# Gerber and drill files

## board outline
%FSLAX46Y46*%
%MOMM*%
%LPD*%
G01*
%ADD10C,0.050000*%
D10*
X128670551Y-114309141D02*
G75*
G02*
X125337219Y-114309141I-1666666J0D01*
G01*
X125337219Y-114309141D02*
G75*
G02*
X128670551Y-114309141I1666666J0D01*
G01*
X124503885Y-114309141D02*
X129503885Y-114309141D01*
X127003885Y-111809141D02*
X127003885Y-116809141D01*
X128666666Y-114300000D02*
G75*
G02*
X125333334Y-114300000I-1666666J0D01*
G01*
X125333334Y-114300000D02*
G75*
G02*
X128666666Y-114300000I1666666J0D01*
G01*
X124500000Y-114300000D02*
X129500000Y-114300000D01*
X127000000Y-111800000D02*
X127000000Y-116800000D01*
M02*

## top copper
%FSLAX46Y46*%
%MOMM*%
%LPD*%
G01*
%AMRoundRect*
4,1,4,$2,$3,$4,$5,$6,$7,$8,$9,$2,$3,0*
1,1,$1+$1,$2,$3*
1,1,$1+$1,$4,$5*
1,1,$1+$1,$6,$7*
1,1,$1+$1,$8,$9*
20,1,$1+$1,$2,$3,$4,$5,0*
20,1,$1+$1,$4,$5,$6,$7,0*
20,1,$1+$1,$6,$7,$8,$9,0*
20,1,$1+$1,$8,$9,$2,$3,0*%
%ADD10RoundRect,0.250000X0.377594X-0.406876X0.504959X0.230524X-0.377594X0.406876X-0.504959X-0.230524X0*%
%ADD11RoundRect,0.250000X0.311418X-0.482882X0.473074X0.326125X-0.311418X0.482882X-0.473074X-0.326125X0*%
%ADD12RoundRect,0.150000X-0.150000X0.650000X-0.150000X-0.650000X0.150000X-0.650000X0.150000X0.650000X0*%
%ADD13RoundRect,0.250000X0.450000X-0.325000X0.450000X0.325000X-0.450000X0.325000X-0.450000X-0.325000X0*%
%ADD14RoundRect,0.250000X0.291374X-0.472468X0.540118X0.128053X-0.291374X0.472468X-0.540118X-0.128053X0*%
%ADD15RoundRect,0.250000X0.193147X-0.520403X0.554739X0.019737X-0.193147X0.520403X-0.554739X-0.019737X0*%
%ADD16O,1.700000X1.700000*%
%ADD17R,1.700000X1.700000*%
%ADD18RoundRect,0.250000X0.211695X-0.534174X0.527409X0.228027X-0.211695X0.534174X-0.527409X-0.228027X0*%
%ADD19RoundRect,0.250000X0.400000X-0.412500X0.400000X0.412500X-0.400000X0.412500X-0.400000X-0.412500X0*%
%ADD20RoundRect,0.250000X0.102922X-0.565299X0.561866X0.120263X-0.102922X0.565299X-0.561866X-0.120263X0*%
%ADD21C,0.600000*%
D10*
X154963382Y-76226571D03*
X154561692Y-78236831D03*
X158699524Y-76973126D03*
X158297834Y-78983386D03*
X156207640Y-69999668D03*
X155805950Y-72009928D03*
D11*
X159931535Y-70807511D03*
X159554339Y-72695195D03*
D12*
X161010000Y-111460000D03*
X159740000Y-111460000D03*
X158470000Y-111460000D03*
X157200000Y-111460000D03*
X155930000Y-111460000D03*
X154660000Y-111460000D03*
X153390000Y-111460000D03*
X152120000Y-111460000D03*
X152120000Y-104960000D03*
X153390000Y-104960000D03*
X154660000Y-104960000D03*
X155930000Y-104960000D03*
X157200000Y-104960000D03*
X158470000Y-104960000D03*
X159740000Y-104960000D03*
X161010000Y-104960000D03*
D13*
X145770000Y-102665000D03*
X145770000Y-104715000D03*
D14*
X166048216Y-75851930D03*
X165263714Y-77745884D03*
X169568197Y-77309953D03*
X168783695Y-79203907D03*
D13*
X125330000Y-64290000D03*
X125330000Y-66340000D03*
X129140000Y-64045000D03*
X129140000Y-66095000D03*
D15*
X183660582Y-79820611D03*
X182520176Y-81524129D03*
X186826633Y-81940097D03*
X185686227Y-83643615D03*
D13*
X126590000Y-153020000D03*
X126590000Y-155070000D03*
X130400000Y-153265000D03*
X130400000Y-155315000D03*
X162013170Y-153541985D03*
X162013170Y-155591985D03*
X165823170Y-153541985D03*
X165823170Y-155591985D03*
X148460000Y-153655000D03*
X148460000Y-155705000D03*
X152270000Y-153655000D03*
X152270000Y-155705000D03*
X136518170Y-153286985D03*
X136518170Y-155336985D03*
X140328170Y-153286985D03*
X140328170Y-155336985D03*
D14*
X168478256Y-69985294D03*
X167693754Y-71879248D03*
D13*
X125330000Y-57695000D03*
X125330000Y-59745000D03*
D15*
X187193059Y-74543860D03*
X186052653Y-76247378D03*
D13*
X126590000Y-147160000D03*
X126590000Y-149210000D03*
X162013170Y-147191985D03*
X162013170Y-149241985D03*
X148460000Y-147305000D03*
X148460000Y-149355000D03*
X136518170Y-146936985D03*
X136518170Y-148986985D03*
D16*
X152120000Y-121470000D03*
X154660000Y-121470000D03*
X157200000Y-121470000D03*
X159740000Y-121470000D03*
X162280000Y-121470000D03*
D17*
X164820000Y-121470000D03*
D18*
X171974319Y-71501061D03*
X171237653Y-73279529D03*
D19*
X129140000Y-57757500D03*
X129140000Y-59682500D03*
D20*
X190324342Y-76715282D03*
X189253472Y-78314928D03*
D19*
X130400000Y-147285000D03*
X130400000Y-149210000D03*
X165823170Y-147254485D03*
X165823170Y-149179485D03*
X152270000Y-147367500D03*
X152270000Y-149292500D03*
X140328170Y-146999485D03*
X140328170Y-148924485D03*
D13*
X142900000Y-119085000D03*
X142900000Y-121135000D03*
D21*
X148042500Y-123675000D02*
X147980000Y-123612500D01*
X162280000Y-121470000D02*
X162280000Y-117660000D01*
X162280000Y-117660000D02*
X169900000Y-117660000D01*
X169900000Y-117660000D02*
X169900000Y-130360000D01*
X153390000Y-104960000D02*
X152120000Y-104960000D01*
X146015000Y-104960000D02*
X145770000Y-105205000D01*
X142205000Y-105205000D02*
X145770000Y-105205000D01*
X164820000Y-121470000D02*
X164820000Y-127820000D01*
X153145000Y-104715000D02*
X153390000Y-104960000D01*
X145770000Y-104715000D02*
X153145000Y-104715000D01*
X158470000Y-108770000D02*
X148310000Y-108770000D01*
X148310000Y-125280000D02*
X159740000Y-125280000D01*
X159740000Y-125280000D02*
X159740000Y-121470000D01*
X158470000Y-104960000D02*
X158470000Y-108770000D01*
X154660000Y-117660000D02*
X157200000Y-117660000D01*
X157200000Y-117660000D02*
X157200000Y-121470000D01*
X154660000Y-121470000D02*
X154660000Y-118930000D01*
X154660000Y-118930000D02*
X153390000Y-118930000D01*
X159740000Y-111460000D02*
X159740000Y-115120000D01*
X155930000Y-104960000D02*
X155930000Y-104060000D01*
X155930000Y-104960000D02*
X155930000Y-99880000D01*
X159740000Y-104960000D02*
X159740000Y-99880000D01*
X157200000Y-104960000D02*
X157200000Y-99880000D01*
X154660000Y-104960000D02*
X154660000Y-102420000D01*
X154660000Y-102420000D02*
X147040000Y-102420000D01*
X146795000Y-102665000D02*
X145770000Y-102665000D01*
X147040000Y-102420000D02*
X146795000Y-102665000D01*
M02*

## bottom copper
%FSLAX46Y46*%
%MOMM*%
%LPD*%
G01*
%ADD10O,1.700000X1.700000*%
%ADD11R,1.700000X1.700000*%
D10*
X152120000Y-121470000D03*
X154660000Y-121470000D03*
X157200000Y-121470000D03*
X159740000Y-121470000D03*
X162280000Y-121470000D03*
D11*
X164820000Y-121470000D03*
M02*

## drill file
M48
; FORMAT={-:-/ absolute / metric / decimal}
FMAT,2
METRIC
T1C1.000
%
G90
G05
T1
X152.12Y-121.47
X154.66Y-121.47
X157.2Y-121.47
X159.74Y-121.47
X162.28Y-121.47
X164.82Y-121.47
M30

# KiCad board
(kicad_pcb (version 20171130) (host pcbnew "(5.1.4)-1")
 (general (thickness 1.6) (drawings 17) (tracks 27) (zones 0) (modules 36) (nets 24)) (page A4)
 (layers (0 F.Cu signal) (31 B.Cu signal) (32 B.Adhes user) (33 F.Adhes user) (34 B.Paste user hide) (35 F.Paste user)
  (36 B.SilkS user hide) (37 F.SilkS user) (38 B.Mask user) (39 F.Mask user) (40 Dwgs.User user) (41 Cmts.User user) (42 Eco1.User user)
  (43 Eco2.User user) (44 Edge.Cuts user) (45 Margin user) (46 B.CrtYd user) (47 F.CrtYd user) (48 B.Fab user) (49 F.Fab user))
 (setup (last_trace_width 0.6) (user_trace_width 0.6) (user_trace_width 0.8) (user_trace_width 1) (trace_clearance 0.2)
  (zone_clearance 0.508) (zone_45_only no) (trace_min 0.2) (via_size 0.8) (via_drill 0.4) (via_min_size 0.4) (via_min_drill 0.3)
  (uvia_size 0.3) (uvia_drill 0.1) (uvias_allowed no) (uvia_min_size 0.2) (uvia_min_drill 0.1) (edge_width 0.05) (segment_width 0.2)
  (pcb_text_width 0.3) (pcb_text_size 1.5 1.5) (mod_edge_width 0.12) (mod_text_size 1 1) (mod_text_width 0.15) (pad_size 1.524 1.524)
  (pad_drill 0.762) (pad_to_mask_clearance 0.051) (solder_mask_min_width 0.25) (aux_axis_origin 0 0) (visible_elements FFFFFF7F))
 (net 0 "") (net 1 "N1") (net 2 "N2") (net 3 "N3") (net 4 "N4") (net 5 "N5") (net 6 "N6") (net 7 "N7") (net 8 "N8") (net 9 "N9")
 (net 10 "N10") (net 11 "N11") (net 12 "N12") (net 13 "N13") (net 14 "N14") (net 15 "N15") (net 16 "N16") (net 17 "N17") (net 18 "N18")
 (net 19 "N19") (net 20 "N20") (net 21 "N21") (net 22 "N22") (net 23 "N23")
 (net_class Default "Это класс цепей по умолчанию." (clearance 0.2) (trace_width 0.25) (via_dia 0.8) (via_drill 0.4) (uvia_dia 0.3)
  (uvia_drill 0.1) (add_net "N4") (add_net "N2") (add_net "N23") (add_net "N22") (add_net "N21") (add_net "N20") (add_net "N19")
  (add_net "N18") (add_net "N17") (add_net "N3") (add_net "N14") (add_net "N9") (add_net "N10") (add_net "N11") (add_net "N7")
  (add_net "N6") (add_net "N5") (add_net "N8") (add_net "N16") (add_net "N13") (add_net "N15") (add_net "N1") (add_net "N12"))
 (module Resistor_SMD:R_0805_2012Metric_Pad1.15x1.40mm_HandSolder (layer F.Cu) (at 154.762537 77.231701 78.7)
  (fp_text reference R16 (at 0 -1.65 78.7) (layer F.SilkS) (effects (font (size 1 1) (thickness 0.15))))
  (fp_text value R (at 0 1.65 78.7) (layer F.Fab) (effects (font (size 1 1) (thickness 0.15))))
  (pad 2 smd roundrect (at 1.025 0 78.7) (size 1.15 1.4) (layers F.Cu F.Paste F.Mask) (roundrect_rratio 0.217391) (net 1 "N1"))
  (pad 1 smd roundrect (at -1.025 0 78.7) (size 1.15 1.4) (layers F.Cu F.Paste F.Mask) (roundrect_rratio 0.217391) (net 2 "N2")))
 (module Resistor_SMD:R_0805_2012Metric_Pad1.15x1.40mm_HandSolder (layer F.Cu) (at 158.498679 77.978256 78.7)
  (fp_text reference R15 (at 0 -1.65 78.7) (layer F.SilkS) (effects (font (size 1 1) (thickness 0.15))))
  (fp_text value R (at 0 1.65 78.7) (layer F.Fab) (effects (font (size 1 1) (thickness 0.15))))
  (pad 2 smd roundrect (at 1.025 0 78.7) (size 1.15 1.4) (layers F.Cu F.Paste F.Mask) (roundrect_rratio 0.217391) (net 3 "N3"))
  (pad 1 smd roundrect (at -1.025 0 78.7) (size 1.15 1.4) (layers F.Cu F.Paste F.Mask) (roundrect_rratio 0.217391) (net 2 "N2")))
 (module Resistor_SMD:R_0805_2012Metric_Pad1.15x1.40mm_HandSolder (layer F.Cu) (at 156.006795 71.004798 78.7)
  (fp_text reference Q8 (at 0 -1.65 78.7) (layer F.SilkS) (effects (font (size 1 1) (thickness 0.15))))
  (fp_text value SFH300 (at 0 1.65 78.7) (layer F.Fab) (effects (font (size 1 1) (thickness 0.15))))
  (pad 2 smd roundrect (at 1.025 0 78.7) (size 1.15 1.4) (layers F.Cu F.Paste F.Mask) (roundrect_rratio 0.217391) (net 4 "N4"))
  (pad 1 smd roundrect (at -1.025 0 78.7) (size 1.15 1.4) (layers F.Cu F.Paste F.Mask) (roundrect_rratio 0.217391) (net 1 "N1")))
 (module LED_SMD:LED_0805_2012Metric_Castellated (layer F.Cu) (at 159.742937 71.751353 78.7)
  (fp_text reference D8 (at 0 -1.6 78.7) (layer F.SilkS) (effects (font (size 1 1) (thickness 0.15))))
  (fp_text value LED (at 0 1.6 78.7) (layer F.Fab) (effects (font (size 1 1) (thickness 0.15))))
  (pad 2 smd roundrect (at 0.9625 0 78.7) (size 1.325 1.3) (layers F.Cu F.Paste F.Mask) (roundrect_rratio 0.192308) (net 4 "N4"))
  (pad 1 smd roundrect (at -0.9625 0 78.7) (size 1.325 1.3) (layers F.Cu F.Paste F.Mask) (roundrect_rratio 0.192308) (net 3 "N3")))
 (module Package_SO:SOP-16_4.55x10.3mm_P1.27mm (layer F.Cu) (at 156.565 108.21 270)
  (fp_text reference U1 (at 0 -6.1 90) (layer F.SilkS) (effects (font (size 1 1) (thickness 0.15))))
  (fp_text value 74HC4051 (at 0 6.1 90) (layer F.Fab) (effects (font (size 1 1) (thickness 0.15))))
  (pad 16 smd roundrect (at 3.25 -4.445 270) (size 1.6 0.6) (layers F.Cu F.Paste F.Mask) (roundrect_rratio 0.25) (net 4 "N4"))
  (pad 15 smd roundrect (at 3.25 -3.175 270) (size 1.6 0.6) (layers F.Cu F.Paste F.Mask) (roundrect_rratio 0.25) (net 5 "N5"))
  (pad 14 smd roundrect (at 3.25 -1.905 270) (size 1.6 0.6) (layers F.Cu F.Paste F.Mask) (roundrect_rratio 0.25) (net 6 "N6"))
  (pad 13 smd roundrect (at 3.25 -0.635 270) (size 1.6 0.6) (layers F.Cu F.Paste F.Mask) (roundrect_rratio 0.25) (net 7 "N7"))
  (pad 12 smd roundrect (at 3.25 0.635 270) (size 1.6 0.6) (layers F.Cu F.Paste F.Mask) (roundrect_rratio 0.25) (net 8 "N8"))
  (pad 11 smd roundrect (at 3.25 1.905 270) (size 1.6 0.6) (layers F.Cu F.Paste F.Mask) (roundrect_rratio 0.25) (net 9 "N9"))
  (pad 10 smd roundrect (at 3.25 3.175 270) (size 1.6 0.6) (layers F.Cu F.Paste F.Mask) (roundrect_rratio 0.25) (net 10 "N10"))
  (pad 9 smd roundrect (at 3.25 4.445 270) (size 1.6 0.6) (layers F.Cu F.Paste F.Mask) (roundrect_rratio 0.25) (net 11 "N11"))
  (pad 8 smd roundrect (at -3.25 4.445 270) (size 1.6 0.6) (layers F.Cu F.Paste F.Mask) (roundrect_rratio 0.25) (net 2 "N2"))
  (pad 7 smd roundrect (at -3.25 3.175 270) (size 1.6 0.6) (layers F.Cu F.Paste F.Mask) (roundrect_rratio 0.25) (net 2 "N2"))
  (pad 6 smd roundrect (at -3.25 1.905 270) (size 1.6 0.6) (layers F.Cu F.Paste F.Mask) (roundrect_rratio 0.25) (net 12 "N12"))
  (pad 5 smd roundrect (at -3.25 0.635 270) (size 1.6 0.6) (layers F.Cu F.Paste F.Mask) (roundrect_rratio 0.25) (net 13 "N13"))
  (pad 4 smd roundrect (at -3.25 -0.635 270) (size 1.6 0.6) (layers F.Cu F.Paste F.Mask) (roundrect_rratio 0.25) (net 1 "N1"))
  (pad 3 smd roundrect (at -3.25 -1.905 270) (size 1.6 0.6) (layers F.Cu F.Paste F.Mask) (roundrect_rratio 0.25) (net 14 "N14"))
  (pad 2 smd roundrect (at -3.25 -3.175 270) (size 1.6 0.6) (layers F.Cu F.Paste F.Mask) (roundrect_rratio 0.25) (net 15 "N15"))
  (pad 1 smd roundrect (at -3.25 -4.445 270) (size 1.6 0.6) (layers F.Cu F.Paste F.Mask) (roundrect_rratio 0.25) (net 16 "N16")))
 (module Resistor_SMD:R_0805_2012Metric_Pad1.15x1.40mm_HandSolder (layer F.Cu) (at 145.77 103.69 90)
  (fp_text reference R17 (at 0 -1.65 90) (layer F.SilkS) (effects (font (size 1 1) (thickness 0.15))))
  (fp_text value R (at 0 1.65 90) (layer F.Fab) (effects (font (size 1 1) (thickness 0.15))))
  (pad 2 smd roundrect (at 1.025 0 90) (size 1.15 1.4) (layers F.Cu F.Paste F.Mask) (roundrect_rratio 0.217391) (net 12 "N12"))
  (pad 1 smd roundrect (at -1.025 0 90) (size 1.15 1.4) (layers F.Cu F.Paste F.Mask) (roundrect_rratio 0.217391) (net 2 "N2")))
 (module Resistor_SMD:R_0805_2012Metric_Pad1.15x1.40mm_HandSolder (layer F.Cu) (at 165.655965 76.798907 67.5)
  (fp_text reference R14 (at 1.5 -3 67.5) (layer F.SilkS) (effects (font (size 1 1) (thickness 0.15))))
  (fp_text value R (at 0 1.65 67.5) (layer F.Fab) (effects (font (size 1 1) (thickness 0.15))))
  (pad 2 smd roundrect (at 1.025 0 67.5) (size 1.15 1.4) (layers F.Cu F.Paste F.Mask) (roundrect_rratio 0.217391) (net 15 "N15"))
  (pad 1 smd roundrect (at -1.025 0 67.5) (size 1.15 1.4) (layers F.Cu F.Paste F.Mask) (roundrect_rratio 0.217391) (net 2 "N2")))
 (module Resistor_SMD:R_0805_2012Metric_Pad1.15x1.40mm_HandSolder (layer F.Cu) (at 169.175946 78.25693 67.5)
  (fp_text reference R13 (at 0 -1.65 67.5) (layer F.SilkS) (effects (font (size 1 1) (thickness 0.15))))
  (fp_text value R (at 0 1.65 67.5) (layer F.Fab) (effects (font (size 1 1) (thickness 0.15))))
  (pad 2 smd roundrect (at 1.025 0 67.5) (size 1.15 1.4) (layers F.Cu F.Paste F.Mask) (roundrect_rratio 0.217391) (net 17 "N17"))
  (pad 1 smd roundrect (at -1.025 0 67.5) (size 1.15 1.4) (layers F.Cu F.Paste F.Mask) (roundrect_rratio 0.217391) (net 2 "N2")))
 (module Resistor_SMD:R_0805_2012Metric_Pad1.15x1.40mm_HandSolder (layer F.Cu) (at 125.33 65.315 90)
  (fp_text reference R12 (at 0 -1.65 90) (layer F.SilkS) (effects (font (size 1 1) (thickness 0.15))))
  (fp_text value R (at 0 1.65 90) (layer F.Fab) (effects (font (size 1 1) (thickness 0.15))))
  (pad 2 smd roundrect (at 1.025 0 90) (size 1.15 1.4) (layers F.Cu F.Paste F.Mask) (roundrect_rratio 0.217391) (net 13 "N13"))
  (pad 1 smd roundrect (at -1.025 0 90) (size 1.15 1.4) (layers F.Cu F.Paste F.Mask) (roundrect_rratio 0.217391) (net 2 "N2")))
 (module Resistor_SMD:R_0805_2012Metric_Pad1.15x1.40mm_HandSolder (layer F.Cu) (at 129.14 65.07 90)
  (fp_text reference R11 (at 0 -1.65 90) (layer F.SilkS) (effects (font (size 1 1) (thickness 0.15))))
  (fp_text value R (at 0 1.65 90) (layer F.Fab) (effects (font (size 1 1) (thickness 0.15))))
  (pad 2 smd roundrect (at 1.025 0 90) (size 1.15 1.4) (layers F.Cu F.Paste F.Mask) (roundrect_rratio 0.217391) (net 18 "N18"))
  (pad 1 smd roundrect (at -1.025 0 90) (size 1.15 1.4) (layers F.Cu F.Paste F.Mask) (roundrect_rratio 0.217391) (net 2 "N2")))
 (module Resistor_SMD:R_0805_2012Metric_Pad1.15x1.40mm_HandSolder (layer F.Cu) (at 183.090379 80.67237 56.2)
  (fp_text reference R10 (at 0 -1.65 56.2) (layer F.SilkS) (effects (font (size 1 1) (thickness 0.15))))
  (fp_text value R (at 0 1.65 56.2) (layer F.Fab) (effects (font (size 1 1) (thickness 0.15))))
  (pad 2 smd roundrect (at 1.025 0 56.2) (size 1.15 1.4) (layers F.Cu F.Paste F.Mask) (roundrect_rratio 0.217391) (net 16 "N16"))
  (pad 1 smd roundrect (at -1.025 0 56.2) (size 1.15 1.4) (layers F.Cu F.Paste F.Mask) (roundrect_rratio 0.217391) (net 2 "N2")))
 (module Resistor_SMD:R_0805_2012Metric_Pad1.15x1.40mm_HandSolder (layer F.Cu) (at 186.25643 82.791856 56.2)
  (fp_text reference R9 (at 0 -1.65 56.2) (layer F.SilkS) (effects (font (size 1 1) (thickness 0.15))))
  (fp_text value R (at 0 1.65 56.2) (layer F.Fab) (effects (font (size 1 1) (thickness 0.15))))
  (pad 2 smd roundrect (at 1.025 0 56.2) (size 1.15 1.4) (layers F.Cu F.Paste F.Mask) (roundrect_rratio 0.217391) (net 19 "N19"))
  (pad 1 smd roundrect (at -1.025 0 56.2) (size 1.15 1.4) (layers F.Cu F.Paste F.Mask) (roundrect_rratio 0.217391) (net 2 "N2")))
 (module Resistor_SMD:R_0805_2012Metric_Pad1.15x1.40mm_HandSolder (layer F.Cu) (at 126.59 154.045 90)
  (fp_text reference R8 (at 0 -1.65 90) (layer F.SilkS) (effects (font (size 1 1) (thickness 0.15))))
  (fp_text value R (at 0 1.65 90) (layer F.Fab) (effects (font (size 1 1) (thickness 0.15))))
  (pad 2 smd roundrect (at 1.025 0 90) (size 1.15 1.4) (layers F.Cu F.Paste F.Mask) (roundrect_rratio 0.217391) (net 8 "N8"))
  (pad 1 smd roundrect (at -1.025 0 90) (size 1.15 1.4) (layers F.Cu F.Paste F.Mask) (roundrect_rratio 0.217391) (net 2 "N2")))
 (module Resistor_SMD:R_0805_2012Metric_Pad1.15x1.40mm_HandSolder (layer F.Cu) (at 130.4 154.29 90)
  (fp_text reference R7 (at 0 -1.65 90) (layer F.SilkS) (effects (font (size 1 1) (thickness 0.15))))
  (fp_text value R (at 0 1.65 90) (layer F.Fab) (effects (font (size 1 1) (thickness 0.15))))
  (pad 2 smd roundrect (at 1.025 0 90) (size 1.15 1.4) (layers F.Cu F.Paste F.Mask) (roundrect_rratio 0.217391) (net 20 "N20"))
  (pad 1 smd roundrect (at -1.025 0 90) (size 1.15 1.4) (layers F.Cu F.Paste F.Mask) (roundrect_rratio 0.217391) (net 2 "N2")))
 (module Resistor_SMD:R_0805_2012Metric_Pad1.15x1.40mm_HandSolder (layer F.Cu) (at 162.01317 154.566985 90)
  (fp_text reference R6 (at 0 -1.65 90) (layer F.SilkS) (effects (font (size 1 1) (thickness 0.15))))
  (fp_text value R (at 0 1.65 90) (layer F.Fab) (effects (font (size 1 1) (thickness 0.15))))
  (pad 2 smd roundrect (at 1.025 0 90) (size 1.15 1.4) (layers F.Cu F.Paste F.Mask) (roundrect_rratio 0.217391) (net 5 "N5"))
  (pad 1 smd roundrect (at -1.025 0 90) (size 1.15 1.4) (layers F.Cu F.Paste F.Mask) (roundrect_rratio 0.217391) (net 2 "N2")))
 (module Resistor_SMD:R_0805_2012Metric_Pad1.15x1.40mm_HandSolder (layer F.Cu) (at 165.82317 154.566985 90)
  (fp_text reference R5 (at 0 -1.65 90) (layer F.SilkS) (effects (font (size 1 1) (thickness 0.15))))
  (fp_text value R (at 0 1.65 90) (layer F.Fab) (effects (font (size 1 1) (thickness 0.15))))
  (pad 2 smd roundrect (at 1.025 0 90) (size 1.15 1.4) (layers F.Cu F.Paste F.Mask) (roundrect_rratio 0.217391) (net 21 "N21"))
  (pad 1 smd roundrect (at -1.025 0 90) (size 1.15 1.4) (layers F.Cu F.Paste F.Mask) (roundrect_rratio 0.217391) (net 2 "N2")))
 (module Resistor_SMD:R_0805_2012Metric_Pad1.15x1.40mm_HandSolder (layer F.Cu) (at 148.46 154.68 90)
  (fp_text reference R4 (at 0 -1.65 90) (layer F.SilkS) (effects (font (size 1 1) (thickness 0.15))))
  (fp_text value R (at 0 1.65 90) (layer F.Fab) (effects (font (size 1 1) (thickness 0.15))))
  (pad 2 smd roundrect (at 1.025 0 90) (size 1.15 1.4) (layers F.Cu F.Paste F.Mask) (roundrect_rratio 0.217391) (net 6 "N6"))
  (pad 1 smd roundrect (at -1.025 0 90) (size 1.15 1.4) (layers F.Cu F.Paste F.Mask) (roundrect_rratio 0.217391) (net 2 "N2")))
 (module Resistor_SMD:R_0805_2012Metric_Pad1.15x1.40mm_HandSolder (layer F.Cu) (at 152.27 154.68 90)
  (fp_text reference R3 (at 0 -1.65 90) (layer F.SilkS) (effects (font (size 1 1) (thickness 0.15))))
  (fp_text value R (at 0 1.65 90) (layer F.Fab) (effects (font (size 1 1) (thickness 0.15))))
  (pad 2 smd roundrect (at 1.025 0 90) (size 1.15 1.4) (layers F.Cu F.Paste F.Mask) (roundrect_rratio 0.217391) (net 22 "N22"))
  (pad 1 smd roundrect (at -1.025 0 90) (size 1.15 1.4) (layers F.Cu F.Paste F.Mask) (roundrect_rratio 0.217391) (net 2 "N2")))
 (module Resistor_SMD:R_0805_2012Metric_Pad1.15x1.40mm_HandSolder (layer F.Cu) (at 136.51817 154.311985 90)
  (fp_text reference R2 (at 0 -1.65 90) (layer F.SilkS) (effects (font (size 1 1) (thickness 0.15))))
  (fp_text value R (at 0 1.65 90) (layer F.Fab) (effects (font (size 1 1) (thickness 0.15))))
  (pad 2 smd roundrect (at 1.025 0 90) (size 1.15 1.4) (layers F.Cu F.Paste F.Mask) (roundrect_rratio 0.217391) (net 7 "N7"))
  (pad 1 smd roundrect (at -1.025 0 90) (size 1.15 1.4) (layers F.Cu F.Paste F.Mask) (roundrect_rratio 0.217391) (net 2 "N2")))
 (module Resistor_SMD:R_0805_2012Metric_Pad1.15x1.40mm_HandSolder (layer F.Cu) (at 140.32817 154.311985 90)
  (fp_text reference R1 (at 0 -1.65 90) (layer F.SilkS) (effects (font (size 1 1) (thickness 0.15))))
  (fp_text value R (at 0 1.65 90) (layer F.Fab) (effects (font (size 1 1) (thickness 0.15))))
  (pad 2 smd roundrect (at 1.025 0 90) (size 1.15 1.4) (layers F.Cu F.Paste F.Mask) (roundrect_rratio 0.217391) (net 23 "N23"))
  (pad 1 smd roundrect (at -1.025 0 90) (size 1.15 1.4) (layers F.Cu F.Paste F.Mask) (roundrect_rratio 0.217391) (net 2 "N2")))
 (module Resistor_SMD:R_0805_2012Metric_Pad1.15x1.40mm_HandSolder (layer F.Cu) (at 168.086005 70.932271 67.5)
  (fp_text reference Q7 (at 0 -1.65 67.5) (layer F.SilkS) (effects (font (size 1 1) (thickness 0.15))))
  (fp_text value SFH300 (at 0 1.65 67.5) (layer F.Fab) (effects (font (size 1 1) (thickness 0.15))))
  (pad 2 smd roundrect (at 1.025 0 67.5) (size 1.15 1.4) (layers F.Cu F.Paste F.Mask) (roundrect_rratio 0.217391) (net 4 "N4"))
  (pad 1 smd roundrect (at -1.025 0 67.5) (size 1.15 1.4) (layers F.Cu F.Paste F.Mask) (roundrect_rratio 0.217391) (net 15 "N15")))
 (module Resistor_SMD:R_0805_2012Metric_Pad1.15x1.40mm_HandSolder (layer F.Cu) (at 125.33 58.72 90)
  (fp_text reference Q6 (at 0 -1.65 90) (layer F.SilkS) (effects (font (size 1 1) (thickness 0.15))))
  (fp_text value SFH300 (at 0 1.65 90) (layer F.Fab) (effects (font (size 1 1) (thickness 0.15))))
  (pad 2 smd roundrect (at 1.025 0 90) (size 1.15 1.4) (layers F.Cu F.Paste F.Mask) (roundrect_rratio 0.217391) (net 4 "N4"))
  (pad 1 smd roundrect (at -1.025 0 90) (size 1.15 1.4) (layers F.Cu F.Paste F.Mask) (roundrect_rratio 0.217391) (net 13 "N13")))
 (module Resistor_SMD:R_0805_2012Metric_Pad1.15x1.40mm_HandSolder (layer F.Cu) (at 186.622856 75.395619 56.2)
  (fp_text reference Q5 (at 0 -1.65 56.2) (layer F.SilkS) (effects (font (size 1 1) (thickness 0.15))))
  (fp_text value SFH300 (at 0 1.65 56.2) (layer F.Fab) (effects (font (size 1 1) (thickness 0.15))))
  (pad 2 smd roundrect (at 1.025 0 56.2) (size 1.15 1.4) (layers F.Cu F.Paste F.Mask) (roundrect_rratio 0.217391) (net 4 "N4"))
  (pad 1 smd roundrect (at -1.025 0 56.2) (size 1.15 1.4) (layers F.Cu F.Paste F.Mask) (roundrect_rratio 0.217391) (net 16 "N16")))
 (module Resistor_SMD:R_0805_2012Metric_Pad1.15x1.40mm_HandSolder (layer F.Cu) (at 126.59 148.185 90)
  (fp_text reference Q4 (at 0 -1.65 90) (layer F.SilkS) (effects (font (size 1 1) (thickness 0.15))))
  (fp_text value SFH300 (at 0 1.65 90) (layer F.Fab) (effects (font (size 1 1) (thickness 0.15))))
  (pad 2 smd roundrect (at 1.025 0 90) (size 1.15 1.4) (layers F.Cu F.Paste F.Mask) (roundrect_rratio 0.217391) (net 4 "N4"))
  (pad 1 smd roundrect (at -1.025 0 90) (size 1.15 1.4) (layers F.Cu F.Paste F.Mask) (roundrect_rratio 0.217391) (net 8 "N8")))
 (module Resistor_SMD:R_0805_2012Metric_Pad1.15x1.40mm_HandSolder (layer F.Cu) (at 162.01317 148.216985 90)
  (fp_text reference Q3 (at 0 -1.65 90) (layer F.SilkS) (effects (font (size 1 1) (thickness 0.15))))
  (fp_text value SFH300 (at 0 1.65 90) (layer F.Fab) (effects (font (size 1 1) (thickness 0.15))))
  (pad 2 smd roundrect (at 1.025 0 90) (size 1.15 1.4) (layers F.Cu F.Paste F.Mask) (roundrect_rratio 0.217391) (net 4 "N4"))
  (pad 1 smd roundrect (at -1.025 0 90) (size 1.15 1.4) (layers F.Cu F.Paste F.Mask) (roundrect_rratio 0.217391) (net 5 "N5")))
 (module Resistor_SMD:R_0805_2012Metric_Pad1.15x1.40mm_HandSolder (layer F.Cu) (at 148.46 148.33 90)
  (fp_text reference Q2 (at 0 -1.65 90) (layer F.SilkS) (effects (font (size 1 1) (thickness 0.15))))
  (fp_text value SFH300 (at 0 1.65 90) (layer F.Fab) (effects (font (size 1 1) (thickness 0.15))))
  (pad 2 smd roundrect (at 1.025 0 90) (size 1.15 1.4) (layers F.Cu F.Paste F.Mask) (roundrect_rratio 0.217391) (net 4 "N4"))
  (pad 1 smd roundrect (at -1.025 0 90) (size 1.15 1.4) (layers F.Cu F.Paste F.Mask) (roundrect_rratio 0.217391) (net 6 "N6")))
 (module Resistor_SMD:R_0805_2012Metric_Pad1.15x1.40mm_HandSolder (layer F.Cu) (at 136.51817 147.961985 90)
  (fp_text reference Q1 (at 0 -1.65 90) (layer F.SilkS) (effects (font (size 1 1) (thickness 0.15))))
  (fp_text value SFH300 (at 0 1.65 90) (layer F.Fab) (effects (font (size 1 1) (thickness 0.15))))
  (pad 2 smd roundrect (at 1.025 0 90) (size 1.15 1.4) (layers F.Cu F.Paste F.Mask) (roundrect_rratio 0.217391) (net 4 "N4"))
  (pad 1 smd roundrect (at -1.025 0 90) (size 1.15 1.4) (layers F.Cu F.Paste F.Mask) (roundrect_rratio 0.217391) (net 7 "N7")))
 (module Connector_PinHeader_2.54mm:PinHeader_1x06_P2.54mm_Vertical (layer F.Cu) (at 164.82 121.47 270)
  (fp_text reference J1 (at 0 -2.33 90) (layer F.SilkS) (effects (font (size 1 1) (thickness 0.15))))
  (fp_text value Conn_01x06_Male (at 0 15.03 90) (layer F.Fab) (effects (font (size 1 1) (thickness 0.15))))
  (pad 6 thru_hole oval (at 0 12.7 270) (size 1.7 1.7) (drill 1) (layers *.Cu *.Mask) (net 11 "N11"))
  (pad 5 thru_hole oval (at 0 10.16 270) (size 1.7 1.7) (drill 1) (layers *.Cu *.Mask) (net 10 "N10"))
  (pad 4 thru_hole oval (at 0 7.62 270) (size 1.7 1.7) (drill 1) (layers *.Cu *.Mask) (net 9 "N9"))
  (pad 3 thru_hole oval (at 0 5.08 270) (size 1.7 1.7) (drill 1) (layers *.Cu *.Mask) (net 14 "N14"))
  (pad 2 thru_hole oval (at 0 2.54 270) (size 1.7 1.7) (drill 1) (layers *.Cu *.Mask) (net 4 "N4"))
  (pad 1 thru_hole rect (at 0 0 270) (size 1.7 1.7) (drill 1) (layers *.Cu *.Mask) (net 2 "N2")))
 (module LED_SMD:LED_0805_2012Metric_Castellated (layer F.Cu) (at 171.605986 72.390295 67.5)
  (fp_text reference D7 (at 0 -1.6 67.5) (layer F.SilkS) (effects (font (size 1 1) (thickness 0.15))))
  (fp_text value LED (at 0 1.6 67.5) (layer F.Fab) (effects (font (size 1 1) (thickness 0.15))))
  (pad 2 smd roundrect (at 0.9625 0 67.5) (size 1.325 1.3) (layers F.Cu F.Paste F.Mask) (roundrect_rratio 0.192308) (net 4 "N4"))
  (pad 1 smd roundrect (at -0.9625 0 67.5) (size 1.325 1.3) (layers F.Cu F.Paste F.Mask) (roundrect_rratio 0.192308) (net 17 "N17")))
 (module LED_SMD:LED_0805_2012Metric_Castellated (layer F.Cu) (at 129.14 58.72 90)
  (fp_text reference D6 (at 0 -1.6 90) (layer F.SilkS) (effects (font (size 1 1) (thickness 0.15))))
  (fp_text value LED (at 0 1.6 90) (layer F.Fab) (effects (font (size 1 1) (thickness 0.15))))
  (pad 2 smd roundrect (at 0.9625 0 90) (size 1.325 1.3) (layers F.Cu F.Paste F.Mask) (roundrect_rratio 0.192308) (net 4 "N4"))
  (pad 1 smd roundrect (at -0.9625 0 90) (size 1.325 1.3) (layers F.Cu F.Paste F.Mask) (roundrect_rratio 0.192308) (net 18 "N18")))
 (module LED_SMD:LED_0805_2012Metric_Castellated (layer F.Cu) (at 189.788907 77.515105 56.2)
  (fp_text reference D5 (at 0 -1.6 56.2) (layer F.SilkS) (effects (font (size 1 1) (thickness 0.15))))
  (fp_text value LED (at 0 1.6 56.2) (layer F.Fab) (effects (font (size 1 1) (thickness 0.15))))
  (pad 2 smd roundrect (at 0.9625 0 56.2) (size 1.325 1.3) (layers F.Cu F.Paste F.Mask) (roundrect_rratio 0.192308) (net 4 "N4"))
  (pad 1 smd roundrect (at -0.9625 0 56.2) (size 1.325 1.3) (layers F.Cu F.Paste F.Mask) (roundrect_rratio 0.192308) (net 19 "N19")))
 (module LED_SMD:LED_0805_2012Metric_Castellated (layer F.Cu) (at 130.4 148.2475 90)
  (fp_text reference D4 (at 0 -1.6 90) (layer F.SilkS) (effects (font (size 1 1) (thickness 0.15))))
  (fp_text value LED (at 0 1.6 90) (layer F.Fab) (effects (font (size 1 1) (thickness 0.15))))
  (pad 2 smd roundrect (at 0.9625 0 90) (size 1.325 1.3) (layers F.Cu F.Paste F.Mask) (roundrect_rratio 0.192308) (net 4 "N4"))
  (pad 1 smd roundrect (at -0.9625 0 90) (size 1.325 1.3) (layers F.Cu F.Paste F.Mask) (roundrect_rratio 0.192308) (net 20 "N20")))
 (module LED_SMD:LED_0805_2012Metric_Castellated (layer F.Cu) (at 165.82317 148.216985 90)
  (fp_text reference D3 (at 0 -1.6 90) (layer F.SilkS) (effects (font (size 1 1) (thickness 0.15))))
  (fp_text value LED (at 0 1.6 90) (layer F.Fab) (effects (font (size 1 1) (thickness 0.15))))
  (pad 2 smd roundrect (at 0.9625 0 90) (size 1.325 1.3) (layers F.Cu F.Paste F.Mask) (roundrect_rratio 0.192308) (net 4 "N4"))
  (pad 1 smd roundrect (at -0.9625 0 90) (size 1.325 1.3) (layers F.Cu F.Paste F.Mask) (roundrect_rratio 0.192308) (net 21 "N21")))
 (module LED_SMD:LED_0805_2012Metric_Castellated (layer F.Cu) (at 152.27 148.33 90)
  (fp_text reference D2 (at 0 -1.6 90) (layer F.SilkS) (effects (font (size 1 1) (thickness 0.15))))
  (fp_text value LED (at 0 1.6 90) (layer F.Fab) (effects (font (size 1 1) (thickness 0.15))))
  (pad 2 smd roundrect (at 0.9625 0 90) (size 1.325 1.3) (layers F.Cu F.Paste F.Mask) (roundrect_rratio 0.192308) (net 4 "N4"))
  (pad 1 smd roundrect (at -0.9625 0 90) (size 1.325 1.3) (layers F.Cu F.Paste F.Mask) (roundrect_rratio 0.192308) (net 22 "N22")))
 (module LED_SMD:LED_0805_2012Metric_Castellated (layer F.Cu) (at 140.32817 147.961985 90)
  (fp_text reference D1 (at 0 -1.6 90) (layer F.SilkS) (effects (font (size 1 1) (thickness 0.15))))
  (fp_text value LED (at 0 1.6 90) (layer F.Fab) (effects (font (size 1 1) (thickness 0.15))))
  (pad 2 smd roundrect (at 0.9625 0 90) (size 1.325 1.3) (layers F.Cu F.Paste F.Mask) (roundrect_rratio 0.192308) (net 4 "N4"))
  (pad 1 smd roundrect (at -0.9625 0 90) (size 1.325 1.3) (layers F.Cu F.Paste F.Mask) (roundrect_rratio 0.192308) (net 23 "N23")))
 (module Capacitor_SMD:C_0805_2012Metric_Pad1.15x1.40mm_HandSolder (layer F.Cu) (at 142.9 120.11 90)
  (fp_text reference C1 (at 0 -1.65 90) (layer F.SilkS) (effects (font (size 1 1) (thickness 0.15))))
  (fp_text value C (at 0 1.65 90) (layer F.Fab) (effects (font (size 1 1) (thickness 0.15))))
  (pad 2 smd roundrect (at 1.025 0 90) (size 1.15 1.4) (layers F.Cu F.Paste F.Mask) (roundrect_rratio 0.217391) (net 2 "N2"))
  (pad 1 smd roundrect (at -1.025 0 90) (size 1.15 1.4) (layers F.Cu F.Paste F.Mask) (roundrect_rratio 0.217391) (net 4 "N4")))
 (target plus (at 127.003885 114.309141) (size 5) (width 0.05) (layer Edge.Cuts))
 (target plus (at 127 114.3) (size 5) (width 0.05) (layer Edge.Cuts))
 (segment (start 148.0425 123.675) (end 147.98 123.6125) (width 0.6) (layer F.Cu) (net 4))
 (segment (start 162.28 121.47) (end 162.28 117.66) (width 0.6) (layer F.Cu) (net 4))
 (segment (start 162.28 117.66) (end 169.9 117.66) (width 0.6) (layer F.Cu) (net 4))
 (segment (start 169.9 117.66) (end 169.9 130.36) (width 0.6) (layer F.Cu) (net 4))
 (segment (start 153.39 104.96) (end 152.12 104.96) (width 0.6) (layer F.Cu) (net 2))
 (segment (start 146.015 104.96) (end 145.77 105.205) (width 0.6) (layer F.Cu) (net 2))
 (segment (start 142.205 105.205) (end 145.77 105.205) (width 0.6) (layer F.Cu) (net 2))
 (segment (start 164.82 121.47) (end 164.82 127.82) (width 0.6) (layer F.Cu) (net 2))
 (segment (start 153.145 104.715) (end 153.39 104.96) (width 0.6) (layer F.Cu) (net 2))
 (segment (start 145.77 104.715) (end 153.145 104.715) (width 0.6) (layer F.Cu) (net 2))
 (segment (start 158.47 108.77) (end 148.31 108.77) (width 0.6) (layer F.Cu) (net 14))
 (segment (start 148.31 125.28) (end 159.74 125.28) (width 0.6) (layer F.Cu) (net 14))
 (segment (start 159.74 125.28) (end 159.74 121.47) (width 0.6) (layer F.Cu) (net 14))
 (segment (start 158.47 104.96) (end 158.47 108.77) (width 0.6) (layer F.Cu) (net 14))
 (segment (start 154.66 117.66) (end 157.2 117.66) (width 0.6) (layer F.Cu) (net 9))
 (segment (start 157.2 117.66) (end 157.2 121.47) (width 0.6) (layer F.Cu) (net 9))
 (segment (start 154.66 121.47) (end 154.66 118.93) (width 0.6) (layer F.Cu) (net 10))
 (segment (start 154.66 118.93) (end 153.39 118.93) (width 0.6) (layer F.Cu) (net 10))
 (segment (start 159.74 111.46) (end 159.74 115.12) (width 0.6) (layer F.Cu) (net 5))
 (segment (start 155.93 104.96) (end 155.93 104.06) (width 0.6) (layer F.Cu) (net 13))
 (segment (start 155.93 104.96) (end 155.93 99.88) (width 0.6) (layer F.Cu) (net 13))
 (segment (start 159.74 104.96) (end 159.74 99.88) (width 0.6) (layer F.Cu) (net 15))
 (segment (start 157.2 104.96) (end 157.2 99.88) (width 0.6) (layer F.Cu) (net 1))
 (segment (start 154.66 104.96) (end 154.66 102.42) (width 0.6) (layer F.Cu) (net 12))
 (segment (start 154.66 102.42) (end 147.04 102.42) (width 0.6) (layer F.Cu) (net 12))
 (segment (start 146.795 102.665) (end 145.77 102.665) (width 0.6) (layer F.Cu) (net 12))
 (segment (start 147.04 102.42) (end 146.795 102.665) (width 0.6) (layer F.Cu) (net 12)))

